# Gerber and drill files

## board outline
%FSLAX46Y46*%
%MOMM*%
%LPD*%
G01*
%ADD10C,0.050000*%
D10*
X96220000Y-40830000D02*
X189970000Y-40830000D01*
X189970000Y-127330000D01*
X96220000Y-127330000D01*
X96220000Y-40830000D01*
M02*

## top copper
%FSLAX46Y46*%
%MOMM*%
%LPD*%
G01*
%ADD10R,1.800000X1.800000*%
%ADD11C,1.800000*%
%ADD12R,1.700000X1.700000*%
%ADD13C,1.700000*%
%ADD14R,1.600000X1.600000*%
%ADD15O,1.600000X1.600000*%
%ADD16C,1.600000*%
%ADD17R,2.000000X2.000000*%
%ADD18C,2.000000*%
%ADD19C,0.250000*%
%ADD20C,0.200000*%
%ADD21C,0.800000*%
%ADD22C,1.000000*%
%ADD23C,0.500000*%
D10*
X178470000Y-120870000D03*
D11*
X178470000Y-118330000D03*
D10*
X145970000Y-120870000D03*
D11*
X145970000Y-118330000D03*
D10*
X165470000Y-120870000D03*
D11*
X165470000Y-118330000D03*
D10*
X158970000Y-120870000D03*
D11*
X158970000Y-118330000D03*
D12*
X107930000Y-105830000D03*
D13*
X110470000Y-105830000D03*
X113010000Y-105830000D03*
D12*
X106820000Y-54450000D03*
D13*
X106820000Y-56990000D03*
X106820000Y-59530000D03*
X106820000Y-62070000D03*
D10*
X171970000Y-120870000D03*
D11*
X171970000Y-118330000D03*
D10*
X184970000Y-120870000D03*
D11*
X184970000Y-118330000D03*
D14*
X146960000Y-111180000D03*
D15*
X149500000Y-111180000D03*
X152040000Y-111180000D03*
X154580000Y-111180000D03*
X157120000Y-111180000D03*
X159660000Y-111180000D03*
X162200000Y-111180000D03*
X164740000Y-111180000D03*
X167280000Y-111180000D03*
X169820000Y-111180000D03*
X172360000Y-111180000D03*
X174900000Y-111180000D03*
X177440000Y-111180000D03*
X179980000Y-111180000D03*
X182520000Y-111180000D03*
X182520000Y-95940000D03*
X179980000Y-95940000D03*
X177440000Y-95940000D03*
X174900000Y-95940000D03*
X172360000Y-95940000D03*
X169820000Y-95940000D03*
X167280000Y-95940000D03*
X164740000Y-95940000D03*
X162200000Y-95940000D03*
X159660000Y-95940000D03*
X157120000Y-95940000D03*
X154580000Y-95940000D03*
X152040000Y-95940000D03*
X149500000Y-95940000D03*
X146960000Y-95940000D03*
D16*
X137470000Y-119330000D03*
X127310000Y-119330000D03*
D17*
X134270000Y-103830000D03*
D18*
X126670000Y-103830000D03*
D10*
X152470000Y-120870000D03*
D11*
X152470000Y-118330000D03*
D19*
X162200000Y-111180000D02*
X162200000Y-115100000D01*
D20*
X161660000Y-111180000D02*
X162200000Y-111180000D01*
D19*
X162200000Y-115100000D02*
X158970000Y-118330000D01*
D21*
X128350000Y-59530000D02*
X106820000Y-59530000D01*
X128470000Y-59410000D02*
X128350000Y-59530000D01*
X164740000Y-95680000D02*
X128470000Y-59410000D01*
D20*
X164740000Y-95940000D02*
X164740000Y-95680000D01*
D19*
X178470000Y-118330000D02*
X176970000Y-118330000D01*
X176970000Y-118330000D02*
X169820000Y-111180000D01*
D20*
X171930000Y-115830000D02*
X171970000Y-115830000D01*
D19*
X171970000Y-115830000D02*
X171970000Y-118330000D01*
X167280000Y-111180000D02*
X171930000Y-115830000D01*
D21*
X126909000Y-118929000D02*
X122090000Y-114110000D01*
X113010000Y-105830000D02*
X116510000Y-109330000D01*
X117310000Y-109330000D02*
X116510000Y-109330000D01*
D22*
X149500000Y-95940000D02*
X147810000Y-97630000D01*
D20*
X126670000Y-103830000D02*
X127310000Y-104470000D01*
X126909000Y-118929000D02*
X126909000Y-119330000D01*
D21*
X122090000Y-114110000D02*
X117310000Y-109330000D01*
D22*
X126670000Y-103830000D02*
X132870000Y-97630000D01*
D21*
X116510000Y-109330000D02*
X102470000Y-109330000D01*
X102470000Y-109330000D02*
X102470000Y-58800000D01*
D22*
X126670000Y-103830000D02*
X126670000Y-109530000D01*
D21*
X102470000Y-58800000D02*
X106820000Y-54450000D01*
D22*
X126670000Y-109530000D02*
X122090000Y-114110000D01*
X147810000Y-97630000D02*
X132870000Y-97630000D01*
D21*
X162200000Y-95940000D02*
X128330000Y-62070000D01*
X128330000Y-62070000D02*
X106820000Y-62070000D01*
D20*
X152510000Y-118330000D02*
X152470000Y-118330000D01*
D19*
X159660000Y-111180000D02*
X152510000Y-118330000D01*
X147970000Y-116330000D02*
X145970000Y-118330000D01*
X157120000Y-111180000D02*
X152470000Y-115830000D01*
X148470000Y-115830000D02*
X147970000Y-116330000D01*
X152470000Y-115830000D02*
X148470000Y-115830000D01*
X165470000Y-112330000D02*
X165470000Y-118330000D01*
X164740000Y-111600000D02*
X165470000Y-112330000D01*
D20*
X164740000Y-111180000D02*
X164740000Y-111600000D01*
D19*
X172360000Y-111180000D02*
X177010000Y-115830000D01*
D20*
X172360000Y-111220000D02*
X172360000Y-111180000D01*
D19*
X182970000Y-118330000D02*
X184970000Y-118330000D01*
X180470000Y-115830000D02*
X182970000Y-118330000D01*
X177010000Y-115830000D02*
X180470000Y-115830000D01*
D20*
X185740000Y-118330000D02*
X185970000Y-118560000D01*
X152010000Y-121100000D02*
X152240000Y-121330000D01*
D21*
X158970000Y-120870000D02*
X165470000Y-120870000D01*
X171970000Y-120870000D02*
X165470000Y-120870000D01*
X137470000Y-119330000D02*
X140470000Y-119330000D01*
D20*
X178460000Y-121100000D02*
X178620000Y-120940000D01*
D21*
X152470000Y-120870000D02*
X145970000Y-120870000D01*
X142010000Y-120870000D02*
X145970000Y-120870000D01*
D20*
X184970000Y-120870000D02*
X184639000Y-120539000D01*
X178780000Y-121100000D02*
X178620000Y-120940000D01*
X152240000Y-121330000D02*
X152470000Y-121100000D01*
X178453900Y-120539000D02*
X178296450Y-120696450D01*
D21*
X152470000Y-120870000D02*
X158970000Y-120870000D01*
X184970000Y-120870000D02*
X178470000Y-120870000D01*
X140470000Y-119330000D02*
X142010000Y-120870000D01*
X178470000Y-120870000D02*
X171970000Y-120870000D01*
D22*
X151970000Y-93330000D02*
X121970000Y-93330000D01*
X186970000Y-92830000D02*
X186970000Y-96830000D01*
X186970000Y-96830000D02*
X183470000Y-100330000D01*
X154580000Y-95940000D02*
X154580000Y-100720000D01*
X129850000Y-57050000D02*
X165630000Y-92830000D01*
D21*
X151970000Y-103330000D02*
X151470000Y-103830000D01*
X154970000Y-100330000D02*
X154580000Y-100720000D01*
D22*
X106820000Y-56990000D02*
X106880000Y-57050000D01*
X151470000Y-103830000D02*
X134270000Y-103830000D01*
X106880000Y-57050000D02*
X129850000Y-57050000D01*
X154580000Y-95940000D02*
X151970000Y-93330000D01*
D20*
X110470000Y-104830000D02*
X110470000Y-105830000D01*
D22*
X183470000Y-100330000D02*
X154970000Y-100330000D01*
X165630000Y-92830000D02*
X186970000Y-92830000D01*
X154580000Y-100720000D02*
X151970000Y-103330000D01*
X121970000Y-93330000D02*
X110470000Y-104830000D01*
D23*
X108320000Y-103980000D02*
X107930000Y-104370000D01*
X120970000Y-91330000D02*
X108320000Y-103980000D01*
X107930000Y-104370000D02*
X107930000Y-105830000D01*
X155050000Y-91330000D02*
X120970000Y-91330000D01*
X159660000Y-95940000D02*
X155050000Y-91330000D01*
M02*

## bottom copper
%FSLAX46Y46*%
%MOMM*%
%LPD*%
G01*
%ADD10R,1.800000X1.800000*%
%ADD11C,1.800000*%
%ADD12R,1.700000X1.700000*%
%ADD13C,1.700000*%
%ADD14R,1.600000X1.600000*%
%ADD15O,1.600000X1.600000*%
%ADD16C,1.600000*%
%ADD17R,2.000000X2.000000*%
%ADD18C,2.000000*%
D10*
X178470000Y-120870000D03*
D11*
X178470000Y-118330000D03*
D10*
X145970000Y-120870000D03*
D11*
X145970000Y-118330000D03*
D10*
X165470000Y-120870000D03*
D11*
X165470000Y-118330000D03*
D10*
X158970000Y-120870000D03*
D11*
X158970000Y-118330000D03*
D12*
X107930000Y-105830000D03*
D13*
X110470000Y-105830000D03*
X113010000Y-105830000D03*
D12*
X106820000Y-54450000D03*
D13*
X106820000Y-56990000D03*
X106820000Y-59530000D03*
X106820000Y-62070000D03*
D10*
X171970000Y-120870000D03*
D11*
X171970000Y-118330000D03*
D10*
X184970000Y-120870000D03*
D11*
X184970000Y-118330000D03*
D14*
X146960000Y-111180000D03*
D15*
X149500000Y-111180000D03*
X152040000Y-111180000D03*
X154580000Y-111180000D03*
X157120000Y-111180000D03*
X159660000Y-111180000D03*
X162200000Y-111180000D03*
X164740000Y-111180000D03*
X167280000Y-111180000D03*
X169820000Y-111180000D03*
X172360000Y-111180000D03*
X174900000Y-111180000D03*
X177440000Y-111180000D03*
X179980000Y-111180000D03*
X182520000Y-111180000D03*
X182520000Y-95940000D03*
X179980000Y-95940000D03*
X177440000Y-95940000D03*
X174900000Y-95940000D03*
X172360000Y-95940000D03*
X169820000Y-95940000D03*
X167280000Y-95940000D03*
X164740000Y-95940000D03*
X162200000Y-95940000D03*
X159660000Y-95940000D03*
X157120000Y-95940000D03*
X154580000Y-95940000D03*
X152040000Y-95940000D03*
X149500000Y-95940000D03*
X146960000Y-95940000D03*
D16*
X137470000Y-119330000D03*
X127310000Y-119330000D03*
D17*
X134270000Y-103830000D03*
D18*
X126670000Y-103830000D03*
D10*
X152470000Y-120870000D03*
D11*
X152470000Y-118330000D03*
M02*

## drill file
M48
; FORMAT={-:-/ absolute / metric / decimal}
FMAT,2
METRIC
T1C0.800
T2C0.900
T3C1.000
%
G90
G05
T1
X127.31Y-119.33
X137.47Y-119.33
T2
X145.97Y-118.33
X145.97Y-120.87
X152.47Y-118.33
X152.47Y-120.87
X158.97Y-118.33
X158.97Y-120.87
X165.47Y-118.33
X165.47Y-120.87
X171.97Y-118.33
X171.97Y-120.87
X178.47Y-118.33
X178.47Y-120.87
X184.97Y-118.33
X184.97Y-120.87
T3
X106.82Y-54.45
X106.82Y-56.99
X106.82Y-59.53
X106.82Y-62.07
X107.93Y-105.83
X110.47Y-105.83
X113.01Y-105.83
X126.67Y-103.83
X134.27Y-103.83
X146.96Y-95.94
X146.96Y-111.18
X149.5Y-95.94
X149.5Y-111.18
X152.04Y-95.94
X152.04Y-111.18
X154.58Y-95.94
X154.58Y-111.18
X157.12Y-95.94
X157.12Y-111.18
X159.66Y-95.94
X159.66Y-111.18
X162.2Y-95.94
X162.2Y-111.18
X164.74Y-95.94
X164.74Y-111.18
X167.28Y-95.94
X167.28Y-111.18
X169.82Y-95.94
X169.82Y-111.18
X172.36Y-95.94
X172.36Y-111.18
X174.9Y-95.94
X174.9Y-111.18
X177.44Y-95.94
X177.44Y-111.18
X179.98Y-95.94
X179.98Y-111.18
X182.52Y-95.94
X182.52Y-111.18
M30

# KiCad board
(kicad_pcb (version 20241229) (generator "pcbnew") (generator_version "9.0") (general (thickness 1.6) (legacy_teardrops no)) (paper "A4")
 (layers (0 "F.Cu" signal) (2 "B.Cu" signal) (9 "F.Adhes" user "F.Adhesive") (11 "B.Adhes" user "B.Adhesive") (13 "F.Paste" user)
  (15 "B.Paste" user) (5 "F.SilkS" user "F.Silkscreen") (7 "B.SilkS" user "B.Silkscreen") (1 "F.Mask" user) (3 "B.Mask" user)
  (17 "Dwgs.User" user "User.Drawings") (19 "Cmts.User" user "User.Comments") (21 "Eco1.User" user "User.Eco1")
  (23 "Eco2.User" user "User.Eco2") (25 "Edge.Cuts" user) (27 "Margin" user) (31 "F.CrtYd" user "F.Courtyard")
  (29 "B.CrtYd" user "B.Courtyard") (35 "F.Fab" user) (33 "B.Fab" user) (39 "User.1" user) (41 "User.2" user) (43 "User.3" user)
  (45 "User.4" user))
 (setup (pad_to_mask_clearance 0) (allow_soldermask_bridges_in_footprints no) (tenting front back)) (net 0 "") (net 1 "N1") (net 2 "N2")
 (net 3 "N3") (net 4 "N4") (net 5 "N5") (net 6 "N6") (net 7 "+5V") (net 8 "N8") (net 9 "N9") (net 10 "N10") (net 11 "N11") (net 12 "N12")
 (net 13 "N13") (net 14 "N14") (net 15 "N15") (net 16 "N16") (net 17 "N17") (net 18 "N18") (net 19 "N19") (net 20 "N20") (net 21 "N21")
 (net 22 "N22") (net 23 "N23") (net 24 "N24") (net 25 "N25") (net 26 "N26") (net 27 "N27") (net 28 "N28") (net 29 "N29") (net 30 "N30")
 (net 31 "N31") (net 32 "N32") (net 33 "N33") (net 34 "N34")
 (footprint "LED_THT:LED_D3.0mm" (layer "F.Cu") (at 178.47 120.87 90)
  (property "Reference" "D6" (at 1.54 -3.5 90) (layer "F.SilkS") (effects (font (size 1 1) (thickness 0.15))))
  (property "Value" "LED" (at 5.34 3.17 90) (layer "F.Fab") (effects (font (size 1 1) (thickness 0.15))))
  (pad "1" thru_hole rect (at 0 0 90) (size 1.8 1.8) (drill 0.9) (layers "*.Cu" "*.Mask") (remove_unused_layers no) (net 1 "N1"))
  (pad "2" thru_hole circle (at 2.54 0 90) (size 1.8 1.8) (drill 0.9) (layers "*.Cu" "*.Mask") (remove_unused_layers no) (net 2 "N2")))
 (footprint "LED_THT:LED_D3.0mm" (layer "F.Cu") (at 145.97 120.87 90)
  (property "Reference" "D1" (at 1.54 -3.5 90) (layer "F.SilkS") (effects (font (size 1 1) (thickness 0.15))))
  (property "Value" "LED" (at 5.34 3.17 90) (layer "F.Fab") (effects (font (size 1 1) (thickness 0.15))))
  (pad "1" thru_hole rect (at 0 0 90) (size 1.8 1.8) (drill 0.9) (layers "*.Cu" "*.Mask") (remove_unused_layers no) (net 1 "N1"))
  (pad "2" thru_hole circle (at 2.54 0 90) (size 1.8 1.8) (drill 0.9) (layers "*.Cu" "*.Mask") (remove_unused_layers no) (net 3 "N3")))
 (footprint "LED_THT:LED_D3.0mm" (layer "F.Cu") (at 165.47 120.87 90)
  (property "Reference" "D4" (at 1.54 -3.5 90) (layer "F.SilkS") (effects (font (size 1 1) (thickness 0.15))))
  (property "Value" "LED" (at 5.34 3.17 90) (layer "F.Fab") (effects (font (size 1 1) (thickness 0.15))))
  (pad "1" thru_hole rect (at 0 0 90) (size 1.8 1.8) (drill 0.9) (layers "*.Cu" "*.Mask") (remove_unused_layers no) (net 1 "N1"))
  (pad "2" thru_hole circle (at 2.54 0 90) (size 1.8 1.8) (drill 0.9) (layers "*.Cu" "*.Mask") (remove_unused_layers no) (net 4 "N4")))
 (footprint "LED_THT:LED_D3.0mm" (layer "F.Cu") (at 158.97 120.87 90)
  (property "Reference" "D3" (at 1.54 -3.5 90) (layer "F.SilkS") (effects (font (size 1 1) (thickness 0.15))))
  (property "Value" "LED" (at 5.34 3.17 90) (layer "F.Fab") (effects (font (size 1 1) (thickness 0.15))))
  (pad "1" thru_hole rect (at 0 0 90) (size 1.8 1.8) (drill 0.9) (layers "*.Cu" "*.Mask") (remove_unused_layers no) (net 1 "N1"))
  (pad "2" thru_hole circle (at 2.54 0 90) (size 1.8 1.8) (drill 0.9) (layers "*.Cu" "*.Mask") (remove_unused_layers no) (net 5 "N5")))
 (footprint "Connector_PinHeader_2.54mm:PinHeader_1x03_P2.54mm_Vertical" (layer "F.Cu") (at 107.93 105.83 90)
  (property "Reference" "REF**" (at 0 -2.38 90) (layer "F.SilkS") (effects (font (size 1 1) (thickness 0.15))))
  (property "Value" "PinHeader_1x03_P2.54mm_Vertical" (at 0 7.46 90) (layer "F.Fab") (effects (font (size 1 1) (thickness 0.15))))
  (pad "1" thru_hole rect (at 0 0 90) (size 1.7 1.7) (drill 1) (layers "*.Cu" "*.Mask") (remove_unused_layers no))
  (pad "2" thru_hole circle (at 0 2.54 90) (size 1.7 1.7) (drill 1) (layers "*.Cu" "*.Mask") (remove_unused_layers no))
  (pad "3" thru_hole circle (at 0 5.08 90) (size 1.7 1.7) (drill 1) (layers "*.Cu" "*.Mask") (remove_unused_layers no)))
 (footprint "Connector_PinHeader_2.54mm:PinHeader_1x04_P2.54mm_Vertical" (layer "F.Cu") (at 106.82 54.45)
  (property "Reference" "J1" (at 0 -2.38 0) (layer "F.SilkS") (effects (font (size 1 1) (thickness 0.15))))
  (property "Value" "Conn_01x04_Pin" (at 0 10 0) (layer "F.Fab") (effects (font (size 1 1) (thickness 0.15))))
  (pad "1" thru_hole rect (at 0 0) (size 1.7 1.7) (drill 1) (layers "*.Cu" "*.Mask") (remove_unused_layers no) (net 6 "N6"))
  (pad "2" thru_hole circle (at 0 2.54) (size 1.7 1.7) (drill 1) (layers "*.Cu" "*.Mask" "F.Paste") (remove_unused_layers no) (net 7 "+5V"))
  (pad "3" thru_hole circle (at 0 5.08) (size 1.7 1.7) (drill 1) (layers "*.Cu" "*.Mask") (remove_unused_layers no) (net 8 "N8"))
  (pad "4" thru_hole circle (at 0 7.62) (size 1.7 1.7) (drill 1) (layers "*.Cu" "*.Mask") (remove_unused_layers no) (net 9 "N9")))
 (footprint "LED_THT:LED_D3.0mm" (layer "F.Cu") (at 171.97 120.87 90)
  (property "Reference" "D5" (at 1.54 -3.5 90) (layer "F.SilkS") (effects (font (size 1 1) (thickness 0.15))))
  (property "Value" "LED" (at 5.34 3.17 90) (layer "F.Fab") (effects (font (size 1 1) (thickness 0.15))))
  (pad "1" thru_hole rect (at 0 0 90) (size 1.8 1.8) (drill 0.9) (layers "*.Cu" "*.Mask") (remove_unused_layers no) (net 1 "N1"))
  (pad "2" thru_hole circle (at 2.54 0 90) (size 1.8 1.8) (drill 0.9) (layers "*.Cu" "*.Mask") (remove_unused_layers no) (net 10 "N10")))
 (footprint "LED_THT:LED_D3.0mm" (layer "F.Cu") (at 184.97 120.87 90)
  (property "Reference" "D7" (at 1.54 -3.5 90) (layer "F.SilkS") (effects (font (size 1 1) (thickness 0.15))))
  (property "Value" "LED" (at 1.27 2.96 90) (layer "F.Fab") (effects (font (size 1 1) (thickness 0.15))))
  (pad "1" thru_hole rect (at 0 0 90) (size 1.8 1.8) (drill 0.9) (layers "*.Cu" "*.Mask") (remove_unused_layers no) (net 1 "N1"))
  (pad "2" thru_hole circle (at 2.54 0 90) (size 1.8 1.8) (drill 0.9) (layers "*.Cu" "*.Mask") (remove_unused_layers no) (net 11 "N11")))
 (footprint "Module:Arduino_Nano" (layer "F.Cu") (at 146.96 111.18 90)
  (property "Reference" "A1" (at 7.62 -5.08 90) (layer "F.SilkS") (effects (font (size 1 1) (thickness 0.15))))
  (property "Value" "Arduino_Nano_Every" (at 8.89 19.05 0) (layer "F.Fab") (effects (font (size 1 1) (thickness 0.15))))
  (pad "1" thru_hole rect (at 0 0 90) (size 1.6 1.6) (drill 1) (layers "*.Cu" "*.Mask") (remove_unused_layers no) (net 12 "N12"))
  (pad "2" thru_hole oval (at 0 2.54 90) (size 1.6 1.6) (drill 1) (layers "*.Cu" "*.Mask") (remove_unused_layers no) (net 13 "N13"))
  (pad "3" thru_hole oval (at 0 5.08 90) (size 1.6 1.6) (drill 1) (layers "*.Cu" "*.Mask") (remove_unused_layers no) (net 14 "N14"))
  (pad "4" thru_hole oval (at 0 7.62 90) (size 1.6 1.6) (drill 1) (layers "*.Cu" "*.Mask") (remove_unused_layers no) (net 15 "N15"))
  (pad "5" thru_hole oval (at 0 10.16 90) (size 1.6 1.6) (drill 1) (layers "*.Cu" "*.Mask") (remove_unused_layers no) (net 3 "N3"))
  (pad "6" thru_hole oval (at 0 12.7 90) (size 1.6 1.6) (drill 1) (layers "*.Cu" "*.Mask") (remove_unused_layers no) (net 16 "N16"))
  (pad "7" thru_hole oval (at 0 15.24 90) (size 1.6 1.6) (drill 1) (layers "*.Cu" "*.Mask") (remove_unused_layers no) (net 5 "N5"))
  (pad "8" thru_hole oval (at 0 17.78 90) (size 1.6 1.6) (drill 1) (layers "*.Cu" "*.Mask") (remove_unused_layers no) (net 4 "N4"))
  (pad "9" thru_hole oval (at 0 20.32 90) (size 1.6 1.6) (drill 1) (layers "*.Cu" "*.Mask") (remove_unused_layers no) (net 10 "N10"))
  (pad "10" thru_hole oval (at 0 22.86 90) (size 1.6 1.6) (drill 1) (layers "*.Cu" "*.Mask") (remove_unused_layers no) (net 2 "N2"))
  (pad "11" thru_hole oval (at 0 25.4 90) (size 1.6 1.6) (drill 1) (layers "*.Cu" "*.Mask") (remove_unused_layers no) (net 11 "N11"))
  (pad "12" thru_hole oval (at 0 27.94 90) (size 1.6 1.6) (drill 1) (layers "*.Cu" "*.Mask") (remove_unused_layers no) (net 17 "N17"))
  (pad "13" thru_hole oval (at 0 30.48 90) (size 1.6 1.6) (drill 1) (layers "*.Cu" "*.Mask") (remove_unused_layers no) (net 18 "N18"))
  (pad "14" thru_hole oval (at 0 33.02 90) (size 1.6 1.6) (drill 1) (layers "*.Cu" "*.Mask") (remove_unused_layers no) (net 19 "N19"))
  (pad "15" thru_hole oval (at 0 35.56 90) (size 1.6 1.6) (drill 1) (layers "*.Cu" "*.Mask") (remove_unused_layers no) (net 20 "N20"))
  (pad "16" thru_hole oval (at 15.24 35.56 90) (size 1.6 1.6) (drill 1) (layers "*.Cu" "*.Mask") (remove_unused_layers no) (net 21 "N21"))
  (pad "17" thru_hole oval (at 15.24 33.02 90) (size 1.6 1.6) (drill 1) (layers "*.Cu" "*.Mask") (remove_unused_layers no) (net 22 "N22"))
  (pad "18" thru_hole oval (at 15.24 30.48 90) (size 1.6 1.6) (drill 1) (layers "*.Cu" "*.Mask") (remove_unused_layers no) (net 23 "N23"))
  (pad "19" thru_hole oval (at 15.24 27.94 90) (size 1.6 1.6) (drill 1) (layers "*.Cu" "*.Mask") (remove_unused_layers no) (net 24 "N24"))
  (pad "20" thru_hole oval (at 15.24 25.4 90) (size 1.6 1.6) (drill 1) (layers "*.Cu" "*.Mask") (remove_unused_layers no) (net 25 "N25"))
  (pad "21" thru_hole oval (at 15.24 22.86 90) (size 1.6 1.6) (drill 1) (layers "*.Cu" "*.Mask") (remove_unused_layers no) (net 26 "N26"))
  (pad "22" thru_hole oval (at 15.24 20.32 90) (size 1.6 1.6) (drill 1) (layers "*.Cu" "*.Mask") (remove_unused_layers no) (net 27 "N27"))
  (pad "23" thru_hole oval (at 15.24 17.78 90) (size 1.6 1.6) (drill 1) (layers "*.Cu" "*.Mask") (remove_unused_layers no) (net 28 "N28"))
  (pad "24" thru_hole oval (at 15.24 15.24 90) (size 1.6 1.6) (drill 1) (layers "*.Cu" "*.Mask") (remove_unused_layers no) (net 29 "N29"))
  (pad "25" thru_hole oval (at 15.24 12.7 90) (size 1.6 1.6) (drill 1) (layers "*.Cu" "*.Mask") (remove_unused_layers no) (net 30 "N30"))
  (pad "26" thru_hole oval (at 15.24 10.16 90) (size 1.6 1.6) (drill 1) (layers "*.Cu" "*.Mask") (remove_unused_layers no) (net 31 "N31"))
  (pad "27" thru_hole oval (at 15.24 7.62 90) (size 1.6 1.6) (drill 1) (layers "*.Cu" "*.Mask") (remove_unused_layers no) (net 7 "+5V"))
  (pad "28" thru_hole oval (at 15.24 5.08 90) (size 1.6 1.6) (drill 1) (layers "*.Cu" "*.Mask") (remove_unused_layers no) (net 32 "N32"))
  (pad "29" thru_hole oval (at 15.24 2.54 90) (size 1.6 1.6) (drill 1) (layers "*.Cu" "*.Mask") (remove_unused_layers no) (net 15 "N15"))
  (pad "30" thru_hole oval (at 15.24 0 90) (size 1.6 1.6) (drill 1) (layers "*.Cu" "*.Mask") (remove_unused_layers no) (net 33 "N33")))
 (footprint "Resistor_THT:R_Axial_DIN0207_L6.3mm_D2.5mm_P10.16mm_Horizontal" (layer "F.Cu") (at 137.47 119.33 180)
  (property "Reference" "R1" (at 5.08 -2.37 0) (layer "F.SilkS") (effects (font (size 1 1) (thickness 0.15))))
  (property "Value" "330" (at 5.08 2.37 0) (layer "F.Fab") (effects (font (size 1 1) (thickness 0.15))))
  (pad "1" thru_hole circle (at 0 0 180) (size 1.6 1.6) (drill 0.8) (layers "*.Cu" "*.Mask") (remove_unused_layers no) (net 1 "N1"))
  (pad "2" thru_hole circle (at 10.16 0 180) (size 1.6 1.6) (drill 0.8) (layers "*.Cu" "*.Mask") (remove_unused_layers no) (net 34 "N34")))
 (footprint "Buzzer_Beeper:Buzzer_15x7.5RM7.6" (layer "F.Cu") (at 134.27 103.83 180)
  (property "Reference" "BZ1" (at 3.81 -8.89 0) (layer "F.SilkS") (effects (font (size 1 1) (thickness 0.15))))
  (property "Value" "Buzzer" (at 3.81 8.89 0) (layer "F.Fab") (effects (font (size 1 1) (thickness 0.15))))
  (pad "1" thru_hole rect (at 0 0 180) (size 2 2) (drill 1) (layers "*.Cu" "*.Mask") (remove_unused_layers no) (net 7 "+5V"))
  (pad "2" thru_hole circle (at 7.6 0 180) (size 2 2) (drill 1) (layers "*.Cu" "*.Mask") (remove_unused_layers no) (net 34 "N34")))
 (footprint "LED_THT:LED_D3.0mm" (layer "F.Cu") (at 152.47 120.87 90)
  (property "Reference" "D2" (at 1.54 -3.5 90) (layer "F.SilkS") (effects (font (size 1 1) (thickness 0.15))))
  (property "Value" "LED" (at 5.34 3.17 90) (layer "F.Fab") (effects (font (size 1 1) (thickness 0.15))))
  (pad "1" thru_hole rect (at 0 0 90) (size 1.8 1.8) (drill 0.9) (layers "*.Cu" "*.Mask") (remove_unused_layers no) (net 1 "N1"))
  (pad "2" thru_hole circle (at 2.54 0 90) (size 1.8 1.8) (drill 0.9) (layers "*.Cu" "*.Mask") (remove_unused_layers no) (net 16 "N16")))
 (gr_rect (start 96.22 40.83) (end 189.97 127.33) (stroke (width 0.05) (type default)) (fill no) (layer "Edge.Cuts"))
 (segment (start 162.2 111.18) (end 162.2 115.1) (width 0.25) (layer "F.Cu") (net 5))
 (segment (start 161.66 111.18) (end 162.2 111.18) (width 0.2) (layer "F.Cu") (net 5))
 (segment (start 162.2 115.1) (end 158.97 118.33) (width 0.25) (layer "F.Cu") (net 5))
 (segment (start 128.35 59.53) (end 106.82 59.53) (width 0.8) (layer "F.Cu") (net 28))
 (segment (start 128.47 59.41) (end 128.35 59.53) (width 0.8) (layer "F.Cu") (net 28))
 (segment (start 164.74 95.68) (end 128.47 59.41) (width 0.8) (layer "F.Cu") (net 28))
 (segment (start 164.74 95.94) (end 164.74 95.68) (width 0.2) (layer "F.Cu") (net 28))
 (segment (start 178.47 118.33) (end 176.97 118.33) (width 0.25) (layer "F.Cu") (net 2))
 (segment (start 176.97 118.33) (end 169.82 111.18) (width 0.25) (layer "F.Cu") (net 2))
 (segment (start 171.93 115.83) (end 171.97 115.83) (width 0.2) (layer "F.Cu") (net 10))
 (segment (start 171.97 115.83) (end 171.97 118.33) (width 0.25) (layer "F.Cu") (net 10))
 (segment (start 167.28 111.18) (end 171.93 115.83) (width 0.25) (layer "F.Cu") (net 10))
 (segment (start 126.909 118.929) (end 122.09 114.11) (width 0.8) (layer "F.Cu") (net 15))
 (segment (start 113.01 105.83) (end 116.51 109.33) (width 0.8) (layer "F.Cu") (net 15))
 (segment (start 117.31 109.33) (end 116.51 109.33) (width 0.8) (layer "F.Cu") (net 15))
 (segment (start 149.5 95.94) (end 147.81 97.63) (width 1) (layer "F.Cu") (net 15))
 (segment (start 126.67 103.83) (end 127.31 104.47) (width 0.2) (layer "F.Cu") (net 15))
 (segment (start 126.909 118.929) (end 126.909 119.33) (width 0.2) (layer "F.Cu") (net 15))
 (segment (start 122.09 114.11) (end 117.31 109.33) (width 0.8) (layer "F.Cu") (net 15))
 (segment (start 126.67 103.83) (end 132.87 97.63) (width 1) (layer "F.Cu") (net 15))
 (segment (start 116.51 109.33) (end 102.47 109.33) (width 0.8) (layer "F.Cu") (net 15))
 (segment (start 102.47 109.33) (end 102.47 58.8) (width 0.8) (layer "F.Cu") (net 15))
 (segment (start 126.67 103.83) (end 126.67 109.53) (width 1) (layer "F.Cu") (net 15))
 (segment (start 102.47 58.8) (end 106.82 54.45) (width 0.8) (layer "F.Cu") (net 15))
 (segment (start 126.67 109.53) (end 122.09 114.11) (width 1) (layer "F.Cu") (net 15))
 (segment (start 147.81 97.63) (end 132.87 97.63) (width 1) (layer "F.Cu") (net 15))
 (segment (start 162.2 95.94) (end 128.33 62.07) (width 0.8) (layer "F.Cu") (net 29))
 (segment (start 128.33 62.07) (end 106.82 62.07) (width 0.8) (layer "F.Cu") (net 29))
 (segment (start 152.51 118.33) (end 152.47 118.33) (width 0.2) (layer "F.Cu") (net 16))
 (segment (start 159.66 111.18) (end 152.51 118.33) (width 0.25) (layer "F.Cu") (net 16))
 (segment (start 147.97 116.33) (end 145.97 118.33) (width 0.25) (layer "F.Cu") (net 3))
 (segment (start 157.12 111.18) (end 152.47 115.83) (width 0.25) (layer "F.Cu") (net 3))
 (segment (start 148.47 115.83) (end 147.97 116.33) (width 0.25) (layer "F.Cu") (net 3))
 (segment (start 152.47 115.83) (end 148.47 115.83) (width 0.25) (layer "F.Cu") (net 3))
 (segment (start 165.47 112.33) (end 165.47 118.33) (width 0.25) (layer "F.Cu") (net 4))
 (segment (start 164.74 111.6) (end 165.47 112.33) (width 0.25) (layer "F.Cu") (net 4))
 (segment (start 164.74 111.18) (end 164.74 111.6) (width 0.2) (layer "F.Cu") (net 4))
 (segment (start 172.36 111.18) (end 177.01 115.83) (width 0.25) (layer "F.Cu") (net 11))
 (segment (start 172.36 111.22) (end 172.36 111.18) (width 0.2) (layer "F.Cu") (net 11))
 (segment (start 182.97 118.33) (end 184.97 118.33) (width 0.25) (layer "F.Cu") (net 11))
 (segment (start 180.47 115.83) (end 182.97 118.33) (width 0.25) (layer "F.Cu") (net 11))
 (segment (start 177.01 115.83) (end 180.47 115.83) (width 0.25) (layer "F.Cu") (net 11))
 (segment (start 185.74 118.33) (end 185.97 118.56) (width 0.2) (layer "F.Cu") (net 11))
 (segment (start 152.01 121.1) (end 152.24 121.33) (width 0.2) (layer "F.Cu") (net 1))
 (segment (start 158.97 120.87) (end 165.47 120.87) (width 0.8) (layer "F.Cu") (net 1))
 (segment (start 171.97 120.87) (end 165.47 120.87) (width 0.8) (layer "F.Cu") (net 1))
 (segment (start 137.47 119.33) (end 140.47 119.33) (width 0.8) (layer "F.Cu") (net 1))
 (segment (start 178.46 121.1) (end 178.62 120.94) (width 0.2) (layer "F.Cu") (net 1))
 (segment (start 152.47 120.87) (end 145.97 120.87) (width 0.8) (layer "F.Cu") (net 1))
 (segment (start 142.01 120.87) (end 145.97 120.87) (width 0.8) (layer "F.Cu") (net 1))
 (segment (start 184.97 120.87) (end 184.639 120.539) (width 0.2) (layer "F.Cu") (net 1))
 (segment (start 178.78 121.1) (end 178.62 120.94) (width 0.2) (layer "F.Cu") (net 1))
 (segment (start 152.24 121.33) (end 152.47 121.1) (width 0.2) (layer "F.Cu") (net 1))
 (segment (start 178.4539 120.539) (end 178.29645 120.69645) (width 0.2) (layer "F.Cu") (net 1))
 (segment (start 152.47 120.87) (end 158.97 120.87) (width 0.8) (layer "F.Cu") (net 1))
 (segment (start 184.97 120.87) (end 178.47 120.87) (width 0.8) (layer "F.Cu") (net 1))
 (segment (start 140.47 119.33) (end 142.01 120.87) (width 0.8) (layer "F.Cu") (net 1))
 (segment (start 178.47 120.87) (end 171.97 120.87) (width 0.8) (layer "F.Cu") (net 1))
 (segment (start 151.97 93.33) (end 121.97 93.33) (width 1) (layer "F.Cu") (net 7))
 (segment (start 186.97 92.83) (end 186.97 96.83) (width 1) (layer "F.Cu") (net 7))
 (segment (start 186.97 96.83) (end 183.47 100.33) (width 1) (layer "F.Cu") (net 7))
 (segment (start 154.58 95.94) (end 154.58 100.72) (width 1) (layer "F.Cu") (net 7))
 (segment (start 129.85 57.05) (end 165.63 92.83) (width 1) (layer "F.Cu") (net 7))
 (segment (start 151.97 103.33) (end 151.47 103.83) (width 0.8) (layer "F.Cu") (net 7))
 (segment (start 154.97 100.33) (end 154.58 100.72) (width 0.8) (layer "F.Cu") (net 7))
 (segment (start 106.82 56.99) (end 106.88 57.05) (width 1) (layer "F.Cu") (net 7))
 (segment (start 151.47 103.83) (end 134.27 103.83) (width 1) (layer "F.Cu") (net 7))
 (segment (start 106.88 57.05) (end 129.85 57.05) (width 1) (layer "F.Cu") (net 7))
 (segment (start 154.58 95.94) (end 151.97 93.33) (width 1) (layer "F.Cu") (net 7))
 (segment (start 110.47 104.83) (end 110.47 105.83) (width 0.2) (layer "F.Cu") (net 7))
 (segment (start 183.47 100.33) (end 154.97 100.33) (width 1) (layer "F.Cu") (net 7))
 (segment (start 165.63 92.83) (end 186.97 92.83) (width 1) (layer "F.Cu") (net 7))
 (segment (start 154.58 100.72) (end 151.97 103.33) (width 1) (layer "F.Cu") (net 7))
 (segment (start 121.97 93.33) (end 110.47 104.83) (width 1) (layer "F.Cu") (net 7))
 (segment (start 108.32 103.98) (end 107.93 104.37) (width 0.5) (layer "F.Cu") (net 30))
 (segment (start 120.97 91.33) (end 108.32 103.98) (width 0.5) (layer "F.Cu") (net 30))
 (segment (start 107.93 104.37) (end 107.93 105.83) (width 0.5) (layer "F.Cu") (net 30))
 (segment (start 155.05 91.33) (end 120.97 91.33) (width 0.5) (layer "F.Cu") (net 30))
 (segment (start 159.66 95.94) (end 155.05 91.33) (width 0.5) (layer "F.Cu") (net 30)))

